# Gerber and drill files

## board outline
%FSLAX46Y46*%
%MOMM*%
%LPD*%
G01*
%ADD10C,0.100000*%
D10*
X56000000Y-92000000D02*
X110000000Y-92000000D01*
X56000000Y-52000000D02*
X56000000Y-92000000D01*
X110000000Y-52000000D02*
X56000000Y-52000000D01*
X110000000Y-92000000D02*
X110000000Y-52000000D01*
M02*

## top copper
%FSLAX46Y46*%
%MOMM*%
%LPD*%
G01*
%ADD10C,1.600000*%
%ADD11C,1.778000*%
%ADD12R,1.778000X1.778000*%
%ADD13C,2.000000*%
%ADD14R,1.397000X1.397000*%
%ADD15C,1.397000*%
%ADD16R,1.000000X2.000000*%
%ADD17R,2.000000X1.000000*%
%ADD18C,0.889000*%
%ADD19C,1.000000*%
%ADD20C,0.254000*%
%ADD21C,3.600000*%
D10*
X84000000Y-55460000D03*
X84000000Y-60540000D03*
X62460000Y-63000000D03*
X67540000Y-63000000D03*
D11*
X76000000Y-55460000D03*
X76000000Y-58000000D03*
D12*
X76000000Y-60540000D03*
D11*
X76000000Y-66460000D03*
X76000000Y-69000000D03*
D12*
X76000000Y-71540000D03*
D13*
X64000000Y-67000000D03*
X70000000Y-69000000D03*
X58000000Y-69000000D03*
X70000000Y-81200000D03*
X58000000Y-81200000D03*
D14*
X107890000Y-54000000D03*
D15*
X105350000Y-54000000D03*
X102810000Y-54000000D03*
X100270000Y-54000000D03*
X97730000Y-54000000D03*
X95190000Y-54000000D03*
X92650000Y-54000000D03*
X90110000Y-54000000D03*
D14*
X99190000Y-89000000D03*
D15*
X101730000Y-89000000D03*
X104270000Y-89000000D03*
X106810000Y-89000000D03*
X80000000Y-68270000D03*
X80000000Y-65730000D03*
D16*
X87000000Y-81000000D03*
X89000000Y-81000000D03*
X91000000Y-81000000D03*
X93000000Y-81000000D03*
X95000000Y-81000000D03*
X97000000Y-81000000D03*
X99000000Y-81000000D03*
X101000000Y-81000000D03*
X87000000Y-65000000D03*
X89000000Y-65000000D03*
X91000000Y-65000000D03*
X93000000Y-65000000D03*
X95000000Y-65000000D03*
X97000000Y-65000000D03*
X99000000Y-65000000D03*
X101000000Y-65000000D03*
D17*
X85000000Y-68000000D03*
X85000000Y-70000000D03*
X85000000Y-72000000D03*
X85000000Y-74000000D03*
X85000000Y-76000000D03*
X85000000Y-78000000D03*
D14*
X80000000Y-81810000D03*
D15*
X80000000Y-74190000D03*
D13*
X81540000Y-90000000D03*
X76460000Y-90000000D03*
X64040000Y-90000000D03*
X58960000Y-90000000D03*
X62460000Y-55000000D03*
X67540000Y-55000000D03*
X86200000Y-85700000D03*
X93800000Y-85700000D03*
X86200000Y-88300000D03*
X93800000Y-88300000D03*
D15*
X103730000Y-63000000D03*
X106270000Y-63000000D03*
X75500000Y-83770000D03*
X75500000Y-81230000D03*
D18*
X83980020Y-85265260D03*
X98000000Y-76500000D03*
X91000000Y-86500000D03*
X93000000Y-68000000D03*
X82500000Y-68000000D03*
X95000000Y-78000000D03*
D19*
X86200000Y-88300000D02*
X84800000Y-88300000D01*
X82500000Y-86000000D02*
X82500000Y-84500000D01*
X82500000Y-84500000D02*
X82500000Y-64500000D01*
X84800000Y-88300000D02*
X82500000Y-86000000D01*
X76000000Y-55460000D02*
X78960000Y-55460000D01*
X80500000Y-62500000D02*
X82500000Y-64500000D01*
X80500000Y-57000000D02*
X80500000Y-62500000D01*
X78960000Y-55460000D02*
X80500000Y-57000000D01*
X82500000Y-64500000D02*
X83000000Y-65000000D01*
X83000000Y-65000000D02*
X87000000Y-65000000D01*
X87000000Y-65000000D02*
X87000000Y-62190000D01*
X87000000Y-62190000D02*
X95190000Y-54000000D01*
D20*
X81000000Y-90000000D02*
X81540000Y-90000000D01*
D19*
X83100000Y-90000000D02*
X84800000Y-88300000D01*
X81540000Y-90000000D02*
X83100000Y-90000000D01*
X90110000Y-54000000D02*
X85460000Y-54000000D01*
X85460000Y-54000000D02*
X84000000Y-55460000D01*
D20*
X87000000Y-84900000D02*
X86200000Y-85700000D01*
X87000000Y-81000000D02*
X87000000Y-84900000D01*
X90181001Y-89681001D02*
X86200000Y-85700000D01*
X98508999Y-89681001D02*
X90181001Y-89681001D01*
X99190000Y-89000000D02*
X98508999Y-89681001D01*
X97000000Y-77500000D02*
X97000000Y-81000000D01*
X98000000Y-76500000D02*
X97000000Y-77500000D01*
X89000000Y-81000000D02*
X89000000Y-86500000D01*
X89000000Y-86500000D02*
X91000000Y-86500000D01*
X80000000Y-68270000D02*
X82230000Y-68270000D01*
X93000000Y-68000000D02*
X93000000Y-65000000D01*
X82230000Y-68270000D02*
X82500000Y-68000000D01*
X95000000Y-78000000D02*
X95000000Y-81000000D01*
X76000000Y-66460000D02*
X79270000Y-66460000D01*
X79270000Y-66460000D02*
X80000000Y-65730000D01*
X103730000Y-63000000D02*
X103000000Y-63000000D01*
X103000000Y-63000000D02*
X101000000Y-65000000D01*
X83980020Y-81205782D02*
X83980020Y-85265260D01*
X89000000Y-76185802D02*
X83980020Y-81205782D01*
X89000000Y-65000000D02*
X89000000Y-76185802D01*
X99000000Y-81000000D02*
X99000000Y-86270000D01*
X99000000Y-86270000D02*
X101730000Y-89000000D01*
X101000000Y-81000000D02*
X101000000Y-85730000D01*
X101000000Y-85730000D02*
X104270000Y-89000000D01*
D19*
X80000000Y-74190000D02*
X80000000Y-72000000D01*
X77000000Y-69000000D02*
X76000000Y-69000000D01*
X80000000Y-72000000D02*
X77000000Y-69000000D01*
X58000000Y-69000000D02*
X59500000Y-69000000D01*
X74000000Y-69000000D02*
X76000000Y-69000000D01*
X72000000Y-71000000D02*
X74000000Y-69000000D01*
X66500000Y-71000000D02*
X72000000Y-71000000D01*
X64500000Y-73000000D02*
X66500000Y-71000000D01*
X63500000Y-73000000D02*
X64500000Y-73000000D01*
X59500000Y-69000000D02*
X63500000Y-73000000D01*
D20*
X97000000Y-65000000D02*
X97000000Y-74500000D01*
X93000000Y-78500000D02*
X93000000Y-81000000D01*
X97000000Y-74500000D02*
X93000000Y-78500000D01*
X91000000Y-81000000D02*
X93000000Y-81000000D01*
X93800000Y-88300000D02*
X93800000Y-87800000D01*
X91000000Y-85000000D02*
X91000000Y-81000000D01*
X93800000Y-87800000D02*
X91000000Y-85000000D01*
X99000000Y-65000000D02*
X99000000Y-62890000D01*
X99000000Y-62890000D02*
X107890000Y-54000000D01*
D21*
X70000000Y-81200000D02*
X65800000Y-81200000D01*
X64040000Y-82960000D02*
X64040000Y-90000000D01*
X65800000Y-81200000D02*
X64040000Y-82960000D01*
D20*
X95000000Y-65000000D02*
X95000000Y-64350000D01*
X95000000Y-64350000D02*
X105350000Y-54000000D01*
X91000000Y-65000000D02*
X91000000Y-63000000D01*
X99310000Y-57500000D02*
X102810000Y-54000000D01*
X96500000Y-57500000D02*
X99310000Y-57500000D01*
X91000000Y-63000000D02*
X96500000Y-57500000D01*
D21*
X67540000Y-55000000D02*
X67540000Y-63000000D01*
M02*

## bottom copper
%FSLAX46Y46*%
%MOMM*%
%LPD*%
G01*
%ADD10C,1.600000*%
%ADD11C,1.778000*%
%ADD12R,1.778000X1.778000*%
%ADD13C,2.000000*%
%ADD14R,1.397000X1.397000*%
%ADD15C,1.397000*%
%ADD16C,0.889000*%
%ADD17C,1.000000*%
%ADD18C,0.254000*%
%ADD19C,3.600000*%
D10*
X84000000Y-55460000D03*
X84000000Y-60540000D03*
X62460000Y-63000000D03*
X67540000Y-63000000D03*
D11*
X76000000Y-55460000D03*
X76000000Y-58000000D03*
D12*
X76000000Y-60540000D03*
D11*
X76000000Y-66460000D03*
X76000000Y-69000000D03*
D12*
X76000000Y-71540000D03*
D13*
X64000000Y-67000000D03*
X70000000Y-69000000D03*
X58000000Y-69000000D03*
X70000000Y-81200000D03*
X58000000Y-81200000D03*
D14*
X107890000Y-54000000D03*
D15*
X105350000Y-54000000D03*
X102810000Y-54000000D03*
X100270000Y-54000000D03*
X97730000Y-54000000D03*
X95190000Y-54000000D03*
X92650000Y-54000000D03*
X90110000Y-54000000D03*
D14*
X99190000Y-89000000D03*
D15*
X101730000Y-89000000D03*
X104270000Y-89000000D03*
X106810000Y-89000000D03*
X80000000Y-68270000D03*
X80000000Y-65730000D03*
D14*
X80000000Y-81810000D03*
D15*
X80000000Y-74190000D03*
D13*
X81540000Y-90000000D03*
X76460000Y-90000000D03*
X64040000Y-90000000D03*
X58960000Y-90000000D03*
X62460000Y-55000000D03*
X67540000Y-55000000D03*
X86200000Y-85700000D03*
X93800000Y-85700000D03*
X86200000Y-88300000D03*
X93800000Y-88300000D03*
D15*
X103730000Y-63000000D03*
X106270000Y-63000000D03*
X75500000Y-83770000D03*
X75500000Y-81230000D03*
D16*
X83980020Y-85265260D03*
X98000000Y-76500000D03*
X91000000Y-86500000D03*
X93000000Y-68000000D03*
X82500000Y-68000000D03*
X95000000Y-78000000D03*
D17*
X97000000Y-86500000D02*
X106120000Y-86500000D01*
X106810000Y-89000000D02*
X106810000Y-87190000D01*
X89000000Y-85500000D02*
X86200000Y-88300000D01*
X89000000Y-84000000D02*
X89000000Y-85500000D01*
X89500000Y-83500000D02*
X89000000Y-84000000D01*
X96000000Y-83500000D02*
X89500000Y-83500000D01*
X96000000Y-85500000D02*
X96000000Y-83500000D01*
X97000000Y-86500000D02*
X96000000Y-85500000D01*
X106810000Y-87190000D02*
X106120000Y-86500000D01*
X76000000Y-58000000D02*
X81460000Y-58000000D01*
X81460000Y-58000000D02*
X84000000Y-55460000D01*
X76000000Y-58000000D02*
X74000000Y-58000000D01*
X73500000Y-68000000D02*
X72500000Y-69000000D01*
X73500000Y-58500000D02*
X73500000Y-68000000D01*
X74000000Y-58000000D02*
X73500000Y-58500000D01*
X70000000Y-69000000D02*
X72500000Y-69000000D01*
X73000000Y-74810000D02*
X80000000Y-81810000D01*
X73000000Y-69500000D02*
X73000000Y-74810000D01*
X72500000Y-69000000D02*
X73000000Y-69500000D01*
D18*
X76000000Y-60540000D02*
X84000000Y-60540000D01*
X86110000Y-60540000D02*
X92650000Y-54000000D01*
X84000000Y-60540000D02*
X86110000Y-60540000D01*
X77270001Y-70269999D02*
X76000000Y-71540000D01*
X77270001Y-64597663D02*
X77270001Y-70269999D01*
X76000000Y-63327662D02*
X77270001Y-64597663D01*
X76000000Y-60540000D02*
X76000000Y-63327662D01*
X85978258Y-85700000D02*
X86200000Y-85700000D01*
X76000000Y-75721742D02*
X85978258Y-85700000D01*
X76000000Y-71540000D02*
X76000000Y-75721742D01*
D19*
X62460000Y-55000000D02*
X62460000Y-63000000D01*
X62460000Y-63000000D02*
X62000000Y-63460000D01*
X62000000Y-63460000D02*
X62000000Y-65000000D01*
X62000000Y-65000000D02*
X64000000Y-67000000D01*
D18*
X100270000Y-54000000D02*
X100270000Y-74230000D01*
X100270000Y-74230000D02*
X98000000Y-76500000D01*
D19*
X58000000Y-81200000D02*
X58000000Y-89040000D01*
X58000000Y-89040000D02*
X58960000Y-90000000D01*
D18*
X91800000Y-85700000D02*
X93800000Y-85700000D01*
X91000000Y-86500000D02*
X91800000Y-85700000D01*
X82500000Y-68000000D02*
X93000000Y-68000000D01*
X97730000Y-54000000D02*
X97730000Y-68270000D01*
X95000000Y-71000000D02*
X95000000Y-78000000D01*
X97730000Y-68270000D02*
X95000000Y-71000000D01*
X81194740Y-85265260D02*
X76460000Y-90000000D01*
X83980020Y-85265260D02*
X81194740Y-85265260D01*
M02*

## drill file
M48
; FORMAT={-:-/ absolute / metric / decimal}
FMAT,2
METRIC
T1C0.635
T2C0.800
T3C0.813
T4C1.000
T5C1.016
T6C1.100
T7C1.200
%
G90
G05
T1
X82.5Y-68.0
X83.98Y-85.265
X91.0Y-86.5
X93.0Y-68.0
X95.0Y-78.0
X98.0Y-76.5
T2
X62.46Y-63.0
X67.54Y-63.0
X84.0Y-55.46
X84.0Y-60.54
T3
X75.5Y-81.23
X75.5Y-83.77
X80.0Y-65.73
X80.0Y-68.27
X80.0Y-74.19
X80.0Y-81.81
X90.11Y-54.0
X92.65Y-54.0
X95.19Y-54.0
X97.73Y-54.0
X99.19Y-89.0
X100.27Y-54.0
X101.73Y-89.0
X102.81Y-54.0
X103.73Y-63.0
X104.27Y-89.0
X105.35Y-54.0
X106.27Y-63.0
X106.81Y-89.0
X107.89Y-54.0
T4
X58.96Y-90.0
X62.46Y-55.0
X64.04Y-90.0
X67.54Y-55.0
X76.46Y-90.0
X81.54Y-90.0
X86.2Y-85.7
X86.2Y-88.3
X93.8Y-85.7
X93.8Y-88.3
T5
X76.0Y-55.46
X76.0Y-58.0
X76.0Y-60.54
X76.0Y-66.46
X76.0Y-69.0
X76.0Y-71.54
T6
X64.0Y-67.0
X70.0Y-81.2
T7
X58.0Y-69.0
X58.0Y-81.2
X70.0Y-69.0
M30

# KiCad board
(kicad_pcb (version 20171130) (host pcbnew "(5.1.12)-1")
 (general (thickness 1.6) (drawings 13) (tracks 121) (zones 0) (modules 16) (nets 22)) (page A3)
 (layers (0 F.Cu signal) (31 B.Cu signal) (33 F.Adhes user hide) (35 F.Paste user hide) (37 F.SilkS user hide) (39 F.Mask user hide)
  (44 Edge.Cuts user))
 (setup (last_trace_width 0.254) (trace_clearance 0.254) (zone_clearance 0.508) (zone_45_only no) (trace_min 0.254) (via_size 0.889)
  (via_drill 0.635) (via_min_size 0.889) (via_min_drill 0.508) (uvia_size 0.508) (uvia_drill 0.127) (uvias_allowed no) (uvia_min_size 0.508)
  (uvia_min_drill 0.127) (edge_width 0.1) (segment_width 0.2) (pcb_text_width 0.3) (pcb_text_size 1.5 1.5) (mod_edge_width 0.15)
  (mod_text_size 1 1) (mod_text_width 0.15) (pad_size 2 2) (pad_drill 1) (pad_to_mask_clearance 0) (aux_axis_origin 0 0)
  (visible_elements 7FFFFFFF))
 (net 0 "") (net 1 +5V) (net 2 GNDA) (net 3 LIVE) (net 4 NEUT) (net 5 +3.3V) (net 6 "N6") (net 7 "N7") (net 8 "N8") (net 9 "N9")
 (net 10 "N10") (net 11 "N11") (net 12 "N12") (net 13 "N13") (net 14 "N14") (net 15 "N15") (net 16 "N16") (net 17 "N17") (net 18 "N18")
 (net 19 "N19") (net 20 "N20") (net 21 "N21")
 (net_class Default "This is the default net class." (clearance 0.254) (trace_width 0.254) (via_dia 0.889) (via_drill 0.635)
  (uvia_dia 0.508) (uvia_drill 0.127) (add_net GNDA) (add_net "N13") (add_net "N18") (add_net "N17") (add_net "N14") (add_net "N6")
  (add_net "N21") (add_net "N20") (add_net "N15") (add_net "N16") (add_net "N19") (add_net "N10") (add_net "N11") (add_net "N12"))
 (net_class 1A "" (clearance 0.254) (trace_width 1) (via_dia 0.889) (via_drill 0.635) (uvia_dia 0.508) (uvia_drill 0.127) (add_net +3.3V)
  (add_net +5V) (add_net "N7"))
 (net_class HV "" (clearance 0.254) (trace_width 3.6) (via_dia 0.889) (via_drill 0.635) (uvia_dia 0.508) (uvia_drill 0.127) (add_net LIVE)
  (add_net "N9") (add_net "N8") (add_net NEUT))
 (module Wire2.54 (layer F.Cu) (at 84 58 270)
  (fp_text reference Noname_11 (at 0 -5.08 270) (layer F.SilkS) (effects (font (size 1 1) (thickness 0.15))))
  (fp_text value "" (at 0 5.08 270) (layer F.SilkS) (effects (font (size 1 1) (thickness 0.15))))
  (pad 1 thru_hole circle (at -2.54 0 270) (size 1.6 1.6) (drill 0.8) (layers *.Cu *.Mask F.SilkS) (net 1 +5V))
  (pad 2 thru_hole circle (at 2.54 0 270) (size 1.6 1.6) (drill 0.8) (layers *.Cu *.Mask F.SilkS) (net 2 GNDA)))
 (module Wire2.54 (layer F.Cu) (at 65 63)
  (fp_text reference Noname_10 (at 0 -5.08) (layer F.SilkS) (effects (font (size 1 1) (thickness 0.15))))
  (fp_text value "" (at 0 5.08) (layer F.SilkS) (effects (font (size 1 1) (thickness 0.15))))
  (pad 1 thru_hole circle (at -2.54 0) (size 1.6 1.6) (drill 0.8) (layers *.Cu *.Mask F.SilkS) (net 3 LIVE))
  (pad 2 thru_hole circle (at 2.54 0) (size 1.6 1.6) (drill 0.8) (layers *.Cu *.Mask F.SilkS) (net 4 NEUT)))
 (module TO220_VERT (layer F.Cu) (at 76 58)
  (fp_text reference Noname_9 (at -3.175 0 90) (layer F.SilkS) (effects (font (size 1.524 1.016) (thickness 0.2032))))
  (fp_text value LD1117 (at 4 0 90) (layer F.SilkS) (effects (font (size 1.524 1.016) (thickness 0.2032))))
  (pad 2 thru_hole circle (at 0 -2.54) (size 1.778 1.778) (drill 1.016) (layers *.Cu *.Mask F.SilkS) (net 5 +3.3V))
  (pad 3 thru_hole circle (at 0 0) (size 1.778 1.778) (drill 1.016) (layers *.Cu *.Mask F.SilkS) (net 1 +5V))
  (pad 1 thru_hole rect (at 0 2.54) (size 1.778 1.778) (drill 1.016) (layers *.Cu *.Mask F.SilkS) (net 2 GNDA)))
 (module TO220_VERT (layer F.Cu) (at 76 69)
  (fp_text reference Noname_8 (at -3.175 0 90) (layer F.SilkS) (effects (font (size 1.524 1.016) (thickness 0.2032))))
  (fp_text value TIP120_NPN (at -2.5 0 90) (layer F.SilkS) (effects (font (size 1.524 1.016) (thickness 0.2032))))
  (pad 2 thru_hole circle (at 0 -2.54) (size 1.778 1.778) (drill 1.016) (layers *.Cu *.Mask F.SilkS) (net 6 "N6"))
  (pad 3 thru_hole circle (at 0 0) (size 1.778 1.778) (drill 1.016) (layers *.Cu *.Mask F.SilkS) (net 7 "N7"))
  (pad 1 thru_hole rect (at 0 2.54) (size 1.778 1.778) (drill 1.016) (layers *.Cu *.Mask F.SilkS) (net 2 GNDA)))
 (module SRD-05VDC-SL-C (layer F.Cu) (at 64 67 270)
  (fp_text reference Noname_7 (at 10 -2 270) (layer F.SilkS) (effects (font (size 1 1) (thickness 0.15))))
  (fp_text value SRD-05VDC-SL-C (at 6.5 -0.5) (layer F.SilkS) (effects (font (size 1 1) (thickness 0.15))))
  (pad 1 thru_hole circle (at 0 0 270) (size 2 2) (drill oval 1.1) (layers *.Cu *.Mask F.SilkS) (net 3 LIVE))
  (pad 3 thru_hole circle (at 2 -6 270) (size 2 2) (drill 1.2) (layers *.Cu *.Mask F.SilkS) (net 1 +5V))
  (pad 2 thru_hole circle (at 2 6 270) (size 2 2) (drill 1.2) (layers *.Cu *.Mask F.SilkS) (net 7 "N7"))
  (pad 5 thru_hole circle (at 14.2 -6 270) (size 2 2) (drill 1.1) (layers *.Cu *.Mask F.SilkS) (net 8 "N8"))
  (pad 4 thru_hole circle (at 14.2 6 270) (size 2 2) (drill 1.2) (layers *.Cu *.Mask F.SilkS) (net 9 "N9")))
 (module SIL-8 (layer F.Cu) (at 99 54 180)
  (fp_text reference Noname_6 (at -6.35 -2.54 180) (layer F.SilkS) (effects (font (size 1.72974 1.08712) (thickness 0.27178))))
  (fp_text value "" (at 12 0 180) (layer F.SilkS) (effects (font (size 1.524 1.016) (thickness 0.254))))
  (pad 1 thru_hole rect (at -8.89 0 180) (size 1.397 1.397) (drill 0.8128) (layers *.Cu *.Mask F.SilkS) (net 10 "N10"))
  (pad 2 thru_hole circle (at -6.35 0 180) (size 1.397 1.397) (drill 0.8128) (layers *.Cu *.Mask F.SilkS) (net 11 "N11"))
  (pad 3 thru_hole circle (at -3.81 0 180) (size 1.397 1.397) (drill 0.8128) (layers *.Cu *.Mask F.SilkS) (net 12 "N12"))
  (pad 4 thru_hole circle (at -1.27 0 180) (size 1.397 1.397) (drill 0.8128) (layers *.Cu *.Mask F.SilkS) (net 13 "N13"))
  (pad 5 thru_hole circle (at 1.27 0 180) (size 1.397 1.397) (drill 0.8128) (layers *.Cu *.Mask F.SilkS) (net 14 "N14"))
  (pad 6 thru_hole circle (at 3.81 0 180) (size 1.397 1.397) (drill 0.8128) (layers *.Cu *.Mask F.SilkS) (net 5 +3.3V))
  (pad 7 thru_hole circle (at 6.35 0 180) (size 1.397 1.397) (drill 0.8128) (layers *.Cu *.Mask F.SilkS) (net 2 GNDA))
  (pad 8 thru_hole circle (at 8.89 0 180) (size 1.397 1.397) (drill 0.8128) (layers *.Cu *.Mask F.SilkS) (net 1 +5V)))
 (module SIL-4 (layer F.Cu) (at 103 89)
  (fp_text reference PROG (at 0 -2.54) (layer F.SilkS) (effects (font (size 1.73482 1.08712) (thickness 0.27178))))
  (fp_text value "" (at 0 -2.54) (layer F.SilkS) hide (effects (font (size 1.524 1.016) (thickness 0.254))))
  (pad 1 thru_hole rect (at -3.81 0) (size 1.397 1.397) (drill 0.8128) (layers *.Cu *.Mask F.SilkS) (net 2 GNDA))
  (pad 2 thru_hole circle (at -1.27 0) (size 1.397 1.397) (drill 0.8128) (layers *.Cu *.Mask F.SilkS) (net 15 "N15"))
  (pad 3 thru_hole circle (at 1.27 0) (size 1.397 1.397) (drill 0.8128) (layers *.Cu *.Mask F.SilkS) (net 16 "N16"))
  (pad 4 thru_hole circle (at 3.81 0) (size 1.397 1.397) (drill 0.8128) (layers *.Cu *.Mask F.SilkS) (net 5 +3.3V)))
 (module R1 (layer F.Cu) (at 80 67 90) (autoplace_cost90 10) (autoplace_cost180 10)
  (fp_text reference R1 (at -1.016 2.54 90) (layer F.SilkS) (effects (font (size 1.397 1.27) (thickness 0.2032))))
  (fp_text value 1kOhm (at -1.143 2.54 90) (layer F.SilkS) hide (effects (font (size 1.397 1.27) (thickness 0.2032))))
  (pad 1 thru_hole circle (at -1.27 0 90) (size 1.397 1.397) (drill 0.8128) (layers *.Cu *.Mask F.SilkS) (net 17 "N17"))
  (pad 2 thru_hole circle (at 1.27 0 90) (size 1.397 1.397) (drill 0.8128) (layers *.Cu *.Mask F.SilkS) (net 6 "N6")))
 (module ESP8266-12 (layer F.Cu) (at 109 81 180)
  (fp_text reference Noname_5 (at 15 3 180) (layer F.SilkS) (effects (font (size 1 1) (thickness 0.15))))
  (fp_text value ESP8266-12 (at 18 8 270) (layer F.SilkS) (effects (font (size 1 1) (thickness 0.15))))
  (pad 15 smd rect (at 22 0 180) (size 1 2) (layers F.Cu F.Paste F.Mask) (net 2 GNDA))
  (pad 16 smd rect (at 20 0 180) (size 1 2) (layers F.Cu F.Paste F.Mask) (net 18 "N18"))
  (pad 17 smd rect (at 18 0 180) (size 1 2) (layers F.Cu F.Paste F.Mask) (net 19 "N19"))
  (pad 18 smd rect (at 16 0 180) (size 1 2) (layers F.Cu F.Paste F.Mask) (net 19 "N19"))
  (pad 19 smd rect (at 14 0 180) (size 1 2) (layers F.Cu F.Paste F.Mask) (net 14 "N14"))
  (pad 20 smd rect (at 12 0 180) (size 1 2) (layers F.Cu F.Paste F.Mask) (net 13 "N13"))
  (pad 21 smd rect (at 10 0 180) (size 1 2) (layers F.Cu F.Paste F.Mask) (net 15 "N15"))
  (pad 22 smd rect (at 8 0 180) (size 1 2) (layers F.Cu F.Paste F.Mask) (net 16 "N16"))
  (pad 8 smd rect (at 22 16 180) (size 1 2) (layers F.Cu F.Paste F.Mask) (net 5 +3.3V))
  (pad 7 smd rect (at 20 16 180) (size 1 2) (layers F.Cu F.Paste F.Mask) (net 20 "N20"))
  (pad 6 smd rect (at 18 16 180) (size 1 2) (layers F.Cu F.Paste F.Mask) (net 12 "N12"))
  (pad 5 smd rect (at 16 16 180) (size 1 2) (layers F.Cu F.Paste F.Mask) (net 17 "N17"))
  (pad 4 smd rect (at 14 16 180) (size 1 2) (layers F.Cu F.Paste F.Mask) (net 11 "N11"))
  (pad 3 smd rect (at 12 16 180) (size 1 2) (layers F.Cu F.Paste F.Mask) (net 19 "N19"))
  (pad 2 smd rect (at 10 16 180) (size 1 2) (layers F.Cu F.Paste F.Mask) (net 10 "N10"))
  (pad 1 smd rect (at 8 16 180) (size 1 2) (layers F.Cu F.Paste F.Mask) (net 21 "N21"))
  (pad 9 smd rect (at 24 13 270) (size 1 2) (layers F.Cu F.Paste F.Mask))
  (pad 10 smd rect (at 24 11 270) (size 1 2) (layers F.Cu F.Paste F.Mask))
  (pad 11 smd rect (at 24 9 270) (size 1 2) (layers F.Cu F.Paste F.Mask))
  (pad 12 smd rect (at 24 7 270) (size 1 2) (layers F.Cu F.Paste F.Mask))
  (pad 13 smd rect (at 24 5 270) (size 1 2) (layers F.Cu F.Paste F.Mask))
  (pad 14 smd rect (at 24 3 270) (size 1 2) (layers F.Cu F.Paste F.Mask)))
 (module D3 (layer F.Cu) (at 80 78 270)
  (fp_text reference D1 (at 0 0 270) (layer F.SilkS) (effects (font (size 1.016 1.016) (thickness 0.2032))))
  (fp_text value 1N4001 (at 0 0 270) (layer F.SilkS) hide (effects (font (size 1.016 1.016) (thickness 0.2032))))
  (pad 2 thru_hole rect (at 3.81 0 270) (size 1.397 1.397) (drill 0.8128) (layers *.Cu *.Mask F.SilkS) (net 1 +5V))
  (pad 1 thru_hole circle (at -3.81 0 270) (size 1.397 1.397) (drill 0.8128) (layers *.Cu *.Mask F.SilkS) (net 7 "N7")))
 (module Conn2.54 (layer F.Cu) (at 79 90 180)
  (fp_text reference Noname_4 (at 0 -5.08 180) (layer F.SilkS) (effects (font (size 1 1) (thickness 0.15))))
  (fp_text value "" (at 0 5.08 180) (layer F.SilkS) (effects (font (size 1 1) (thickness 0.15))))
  (pad 1 thru_hole circle (at -2.54 0 180) (size 2 2) (drill 1) (layers *.Cu *.Mask F.SilkS) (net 5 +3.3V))
  (pad 2 thru_hole circle (at 2.54 0 180) (size 2 2) (drill 1) (layers *.Cu *.Mask F.SilkS) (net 20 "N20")))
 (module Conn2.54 (layer F.Cu) (at 61.5 90 180)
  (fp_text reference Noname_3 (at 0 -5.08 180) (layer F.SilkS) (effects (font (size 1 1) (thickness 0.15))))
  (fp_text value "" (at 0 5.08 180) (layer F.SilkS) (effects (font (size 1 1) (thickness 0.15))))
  (pad 1 thru_hole circle (at -2.54 0 180) (size 2 2) (drill 1) (layers *.Cu *.Mask F.SilkS) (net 8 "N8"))
  (pad 2 thru_hole circle (at 2.54 0 180) (size 2 2) (drill 1) (layers *.Cu *.Mask F.SilkS) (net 9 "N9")))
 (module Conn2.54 (layer F.Cu) (at 65 55)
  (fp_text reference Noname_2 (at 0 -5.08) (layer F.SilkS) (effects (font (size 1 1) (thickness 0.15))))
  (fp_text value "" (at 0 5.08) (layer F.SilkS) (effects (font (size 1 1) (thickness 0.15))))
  (pad 1 thru_hole circle (at -2.54 0) (size 2 2) (drill 1) (layers *.Cu *.Mask F.SilkS) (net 3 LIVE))
  (pad 2 thru_hole circle (at 2.54 0) (size 2 2) (drill 1) (layers *.Cu *.Mask F.SilkS) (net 4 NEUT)))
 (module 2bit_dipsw (layer F.Cu) (at 90 87 270)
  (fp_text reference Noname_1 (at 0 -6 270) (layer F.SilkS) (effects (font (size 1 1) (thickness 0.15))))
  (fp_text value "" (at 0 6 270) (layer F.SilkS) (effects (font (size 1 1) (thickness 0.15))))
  (pad 1 thru_hole circle (at -1.3 3.8 270) (size 2 2) (drill 1) (layers *.Cu *.Mask F.SilkS) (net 2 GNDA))
  (pad 2 thru_hole circle (at -1.3 -3.8 270) (size 2 2) (drill 1) (layers *.Cu *.Mask F.SilkS) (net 18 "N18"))
  (pad 3 thru_hole circle (at 1.3 3.8 270) (size 2 2) (drill 1) (layers *.Cu *.Mask F.SilkS) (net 5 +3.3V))
  (pad 4 thru_hole circle (at 1.3 -3.8 270) (size 2 2) (drill 1) (layers *.Cu *.Mask F.SilkS) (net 19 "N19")))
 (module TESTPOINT (layer F.Cu) (at 105 63)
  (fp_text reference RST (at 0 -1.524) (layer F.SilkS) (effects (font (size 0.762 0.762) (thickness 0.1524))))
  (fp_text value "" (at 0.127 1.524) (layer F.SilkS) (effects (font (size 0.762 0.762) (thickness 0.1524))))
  (pad 1 thru_hole circle (at -1.27 0) (size 1.397 1.397) (drill 0.8128) (layers *.Cu *.Mask F.SilkS))
  (pad 1 thru_hole circle (at 1.27 0) (size 1.397 1.397) (drill 0.8128) (layers *.Cu *.Mask F.SilkS)))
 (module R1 (layer F.Cu) (at 75.5 82.5 90) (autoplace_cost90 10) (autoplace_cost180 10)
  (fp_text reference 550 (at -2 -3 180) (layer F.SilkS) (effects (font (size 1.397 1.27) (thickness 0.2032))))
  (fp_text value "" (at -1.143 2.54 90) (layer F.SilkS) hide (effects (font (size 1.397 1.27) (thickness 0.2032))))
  (pad 1 thru_hole circle (at -1.27 0 90) (size 1.397 1.397) (drill 0.8128) (layers *.Cu *.Mask F.SilkS))
  (pad 2 thru_hole circle (at 1.27 0 90) (size 1.397 1.397) (drill 0.8128) (layers *.Cu *.Mask F.SilkS)))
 (gr_line (start 56 92) (end 110 92) (angle 90) (layer Edge.Cuts) (width 0.1))
 (gr_line (start 56 52) (end 56 92) (angle 90) (layer Edge.Cuts) (width 0.1))
 (gr_line (start 110 52) (end 56 52) (angle 90) (layer Edge.Cuts) (width 0.1))
 (gr_line (start 110 92) (end 110 52) (angle 90) (layer Edge.Cuts) (width 0.1))
 (via (at 83.98002 85.26526) (size 0.889) (drill 0.635) (layers F.Cu B.Cu) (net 20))
 (segment (start 86.2 88.3) (end 84.8 88.3) (width 1) (layer F.Cu) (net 5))
 (segment (start 82.5 86) (end 82.5 84.5) (width 1) (layer F.Cu) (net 5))
 (segment (start 82.5 84.5) (end 82.5 64.5) (width 1) (layer F.Cu) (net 5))
 (segment (start 84.8 88.3) (end 82.5 86) (width 1) (layer F.Cu) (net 5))
 (segment (start 97 86.5) (end 106.12 86.5) (width 1) (layer B.Cu) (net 5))
 (segment (start 76 55.46) (end 78.96 55.46) (width 1) (layer F.Cu) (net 5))
 (segment (start 80.5 62.5) (end 82.5 64.5) (width 1) (layer F.Cu) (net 5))
 (segment (start 80.5 57) (end 80.5 62.5) (width 1) (layer F.Cu) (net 5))
 (segment (start 78.96 55.46) (end 80.5 57) (width 1) (layer F.Cu) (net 5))
 (segment (start 82.5 64.5) (end 83 65) (width 1) (layer F.Cu) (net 5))
 (segment (start 83 65) (end 87 65) (width 1) (layer F.Cu) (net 5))
 (segment (start 106.81 89) (end 106.81 87.19) (width 1) (layer B.Cu) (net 5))
 (segment (start 89 85.5) (end 86.2 88.3) (width 1) (layer B.Cu) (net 5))
 (segment (start 89 84) (end 89 85.5) (width 1) (layer B.Cu) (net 5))
 (segment (start 89.5 83.5) (end 89 84) (width 1) (layer B.Cu) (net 5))
 (segment (start 96 83.5) (end 89.5 83.5) (width 1) (layer B.Cu) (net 5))
 (segment (start 96 85.5) (end 96 83.5) (width 1) (layer B.Cu) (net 5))
 (segment (start 97 86.5) (end 96 85.5) (width 1) (layer B.Cu) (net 5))
 (segment (start 106.81 87.19) (end 106.12 86.5) (width 1) (layer B.Cu) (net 5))
 (segment (start 87 65) (end 87 62.19) (width 1) (layer F.Cu) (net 5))
 (segment (start 87 62.19) (end 95.19 54) (width 1) (layer F.Cu) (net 5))
 (segment (start 81 90) (end 81.54 90) (width 0.254) (layer F.Cu) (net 5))
 (segment (start 83.1 90) (end 84.8 88.3) (width 1) (layer F.Cu) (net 5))
 (segment (start 81.54 90) (end 83.1 90) (width 1) (layer F.Cu) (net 5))
 (segment (start 76 58) (end 81.46 58) (width 1) (layer B.Cu) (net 1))
 (segment (start 81.46 58) (end 84 55.46) (width 1) (layer B.Cu) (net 1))
 (segment (start 76 58) (end 74 58) (width 1) (layer B.Cu) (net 1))
 (segment (start 73.5 68) (end 72.5 69) (width 1) (layer B.Cu) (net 1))
 (segment (start 73.5 58.5) (end 73.5 68) (width 1) (layer B.Cu) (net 1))
 (segment (start 74 58) (end 73.5 58.5) (width 1) (layer B.Cu) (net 1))
 (segment (start 90.11 54) (end 85.46 54) (width 1) (layer F.Cu) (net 1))
 (segment (start 85.46 54) (end 84 55.46) (width 1) (layer F.Cu) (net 1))
 (segment (start 70 69) (end 72.5 69) (width 1) (layer B.Cu) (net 1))
 (segment (start 73 74.81) (end 80 81.81) (width 1) (layer B.Cu) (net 1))
 (segment (start 73 69.5) (end 73 74.81) (width 1) (layer B.Cu) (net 1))
 (segment (start 72.5 69) (end 73 69.5) (width 1) (layer B.Cu) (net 1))
 (segment (start 76 60.54) (end 84 60.54) (width 0.254) (layer B.Cu) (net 2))
 (segment (start 86.11 60.54) (end 92.65 54) (width 0.254) (layer B.Cu) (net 2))
 (segment (start 84 60.54) (end 86.11 60.54) (width 0.254) (layer B.Cu) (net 2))
 (segment (start 77.270001 70.269999) (end 76 71.54) (width 0.254) (layer B.Cu) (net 2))
 (segment (start 77.270001 64.597663) (end 77.270001 70.269999) (width 0.254) (layer B.Cu) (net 2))
 (segment (start 76 63.327662) (end 77.270001 64.597663) (width 0.254) (layer B.Cu) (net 2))
 (segment (start 76 60.54) (end 76 63.327662) (width 0.254) (layer B.Cu) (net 2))
 (segment (start 85.978258 85.7) (end 86.2 85.7) (width 0.254) (layer B.Cu) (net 2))
 (segment (start 76 75.721742) (end 85.978258 85.7) (width 0.254) (layer B.Cu) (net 2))
 (segment (start 76 71.54) (end 76 75.721742) (width 0.254) (layer B.Cu) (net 2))
 (segment (start 87 84.9) (end 86.2 85.7) (width 0.254) (layer F.Cu) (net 2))
 (segment (start 87 81) (end 87 84.9) (width 0.254) (layer F.Cu) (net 2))
 (segment (start 90.181001 89.681001) (end 86.2 85.7) (width 0.254) (layer F.Cu) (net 2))
 (segment (start 98.508999 89.681001) (end 90.181001 89.681001) (width 0.254) (layer F.Cu) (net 2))
 (segment (start 99.19 89) (end 98.508999 89.681001) (width 0.254) (layer F.Cu) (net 2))
 (segment (start 62.46 55) (end 62.46 63) (width 3.6) (layer B.Cu) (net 3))
 (segment (start 62.46 63) (end 62 63.46) (width 3.6) (layer B.Cu) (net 3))
 (segment (start 62 63.46) (end 62 65) (width 3.6) (layer B.Cu) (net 3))
 (segment (start 62 65) (end 64 67) (width 3.6) (layer B.Cu) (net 3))
 (segment (start 100.27 54) (end 100.27 74.23) (width 0.254) (layer B.Cu) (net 13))
 (segment (start 97 77.5) (end 97 81) (width 0.254) (layer F.Cu) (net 13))
 (segment (start 98 76.5) (end 97 77.5) (width 0.254) (layer F.Cu) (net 13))
 (segment (start 100.27 74.23) (end 98 76.5) (width 0.254) (layer B.Cu) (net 13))
 (via (at 98 76.5) (size 0.889) (layers F.Cu B.Cu) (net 13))
 (segment (start 58 81.2) (end 58 89.04) (width 3.6) (layer B.Cu) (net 9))
 (segment (start 58 89.04) (end 58.96 90) (width 3.6) (layer B.Cu) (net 9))
 (segment (start 89 81) (end 89 86.5) (width 0.254) (layer F.Cu) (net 18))
 (segment (start 91.8 85.7) (end 93.8 85.7) (width 0.254) (layer B.Cu) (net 18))
 (segment (start 91 86.5) (end 91.8 85.7) (width 0.254) (layer B.Cu) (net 18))
 (segment (start 89 86.5) (end 91 86.5) (width 0.254) (layer F.Cu) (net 18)) (via (at 91 86.5) (size 0.889) (layers F.Cu B.Cu) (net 18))
 (segment (start 80 68.27) (end 82.23 68.27) (width 0.254) (layer F.Cu) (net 17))
 (segment (start 93 68) (end 93 65) (width 0.254) (layer F.Cu) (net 17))
 (segment (start 82.5 68) (end 93 68) (width 0.254) (layer B.Cu) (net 17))
 (segment (start 82.23 68.27) (end 82.5 68) (width 0.254) (layer F.Cu) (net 17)) (via (at 93 68) (size 0.889) (layers F.Cu B.Cu) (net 17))
 (via (at 82.5 68) (size 0.889) (layers F.Cu B.Cu) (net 17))
 (segment (start 97.73 54) (end 97.73 68.27) (width 0.254) (layer B.Cu) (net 14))
 (segment (start 95 78) (end 95 81) (width 0.254) (layer F.Cu) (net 14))
 (segment (start 95 71) (end 95 78) (width 0.254) (layer B.Cu) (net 14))
 (segment (start 97.73 68.27) (end 95 71) (width 0.254) (layer B.Cu) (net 14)) (via (at 95 78) (size 0.889) (layers F.Cu B.Cu) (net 14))
 (segment (start 76 66.46) (end 79.27 66.46) (width 0.254) (layer F.Cu) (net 6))
 (segment (start 79.27 66.46) (end 80 65.73) (width 0.254) (layer F.Cu) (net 6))
 (segment (start 103.73 63) (end 103 63) (width 0.254) (layer F.Cu) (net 21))
 (segment (start 103 63) (end 101 65) (width 0.254) (layer F.Cu) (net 21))
 (segment (start 83.98002 81.205782) (end 83.98002 85.26526) (width 0.254) (layer F.Cu) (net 20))
 (segment (start 89 76.185802) (end 83.98002 81.205782) (width 0.254) (layer F.Cu) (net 20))
 (segment (start 89 65) (end 89 76.185802) (width 0.254) (layer F.Cu) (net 20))
 (segment (start 81.19474 85.26526) (end 76.46 90) (width 0.254) (layer B.Cu) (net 20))
 (segment (start 83.98002 85.26526) (end 81.19474 85.26526) (width 0.254) (layer B.Cu) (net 20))
 (segment (start 99 81) (end 99 86.27) (width 0.254) (layer F.Cu) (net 15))
 (segment (start 99 86.27) (end 101.73 89) (width 0.254) (layer F.Cu) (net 15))
 (segment (start 101 81) (end 101 85.73) (width 0.254) (layer F.Cu) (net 16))
 (segment (start 101 85.73) (end 104.27 89) (width 0.254) (layer F.Cu) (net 16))
 (segment (start 80 74.19) (end 80 72) (width 1) (layer F.Cu) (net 7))
 (segment (start 77 69) (end 76 69) (width 1) (layer F.Cu) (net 7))
 (segment (start 80 72) (end 77 69) (width 1) (layer F.Cu) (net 7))
 (segment (start 58 69) (end 59.5 69) (width 1) (layer F.Cu) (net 7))
 (segment (start 74 69) (end 76 69) (width 1) (layer F.Cu) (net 7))
 (segment (start 72 71) (end 74 69) (width 1) (layer F.Cu) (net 7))
 (segment (start 66.5 71) (end 72 71) (width 1) (layer F.Cu) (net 7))
 (segment (start 64.5 73) (end 66.5 71) (width 1) (layer F.Cu) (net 7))
 (segment (start 63.5 73) (end 64.5 73) (width 1) (layer F.Cu) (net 7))
 (segment (start 59.5 69) (end 63.5 73) (width 1) (layer F.Cu) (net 7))
 (segment (start 97 65) (end 97 74.5) (width 0.254) (layer F.Cu) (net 19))
 (segment (start 93 78.5) (end 93 81) (width 0.254) (layer F.Cu) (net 19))
 (segment (start 97 74.5) (end 93 78.5) (width 0.254) (layer F.Cu) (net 19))
 (segment (start 91 81) (end 93 81) (width 0.254) (layer F.Cu) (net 19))
 (segment (start 93.8 88.3) (end 93.8 87.8) (width 0.254) (layer F.Cu) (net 19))
 (segment (start 91 85) (end 91 81) (width 0.254) (layer F.Cu) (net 19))
 (segment (start 93.8 87.8) (end 91 85) (width 0.254) (layer F.Cu) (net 19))
 (segment (start 99 65) (end 99 62.89) (width 0.254) (layer F.Cu) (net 10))
 (segment (start 99 62.89) (end 107.89 54) (width 0.254) (layer F.Cu) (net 10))
 (segment (start 70 81.2) (end 65.8 81.2) (width 3.6) (layer F.Cu) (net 8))
 (segment (start 64.04 82.96) (end 64.04 90) (width 3.6) (layer F.Cu) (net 8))
 (segment (start 65.8 81.2) (end 64.04 82.96) (width 3.6) (layer F.Cu) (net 8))
 (segment (start 95 65) (end 95 64.35) (width 0.254) (layer F.Cu) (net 11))
 (segment (start 95 64.35) (end 105.35 54) (width 0.254) (layer F.Cu) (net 11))
 (segment (start 91 65) (end 91 63) (width 0.254) (layer F.Cu) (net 12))
 (segment (start 99.31 57.5) (end 102.81 54) (width 0.254) (layer F.Cu) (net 12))
 (segment (start 96.5 57.5) (end 99.31 57.5) (width 0.254) (layer F.Cu) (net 12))
 (segment (start 91 63) (end 96.5 57.5) (width 0.254) (layer F.Cu) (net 12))
 (segment (start 67.54 55) (end 67.54 63) (width 3.6) (layer F.Cu) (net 4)))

